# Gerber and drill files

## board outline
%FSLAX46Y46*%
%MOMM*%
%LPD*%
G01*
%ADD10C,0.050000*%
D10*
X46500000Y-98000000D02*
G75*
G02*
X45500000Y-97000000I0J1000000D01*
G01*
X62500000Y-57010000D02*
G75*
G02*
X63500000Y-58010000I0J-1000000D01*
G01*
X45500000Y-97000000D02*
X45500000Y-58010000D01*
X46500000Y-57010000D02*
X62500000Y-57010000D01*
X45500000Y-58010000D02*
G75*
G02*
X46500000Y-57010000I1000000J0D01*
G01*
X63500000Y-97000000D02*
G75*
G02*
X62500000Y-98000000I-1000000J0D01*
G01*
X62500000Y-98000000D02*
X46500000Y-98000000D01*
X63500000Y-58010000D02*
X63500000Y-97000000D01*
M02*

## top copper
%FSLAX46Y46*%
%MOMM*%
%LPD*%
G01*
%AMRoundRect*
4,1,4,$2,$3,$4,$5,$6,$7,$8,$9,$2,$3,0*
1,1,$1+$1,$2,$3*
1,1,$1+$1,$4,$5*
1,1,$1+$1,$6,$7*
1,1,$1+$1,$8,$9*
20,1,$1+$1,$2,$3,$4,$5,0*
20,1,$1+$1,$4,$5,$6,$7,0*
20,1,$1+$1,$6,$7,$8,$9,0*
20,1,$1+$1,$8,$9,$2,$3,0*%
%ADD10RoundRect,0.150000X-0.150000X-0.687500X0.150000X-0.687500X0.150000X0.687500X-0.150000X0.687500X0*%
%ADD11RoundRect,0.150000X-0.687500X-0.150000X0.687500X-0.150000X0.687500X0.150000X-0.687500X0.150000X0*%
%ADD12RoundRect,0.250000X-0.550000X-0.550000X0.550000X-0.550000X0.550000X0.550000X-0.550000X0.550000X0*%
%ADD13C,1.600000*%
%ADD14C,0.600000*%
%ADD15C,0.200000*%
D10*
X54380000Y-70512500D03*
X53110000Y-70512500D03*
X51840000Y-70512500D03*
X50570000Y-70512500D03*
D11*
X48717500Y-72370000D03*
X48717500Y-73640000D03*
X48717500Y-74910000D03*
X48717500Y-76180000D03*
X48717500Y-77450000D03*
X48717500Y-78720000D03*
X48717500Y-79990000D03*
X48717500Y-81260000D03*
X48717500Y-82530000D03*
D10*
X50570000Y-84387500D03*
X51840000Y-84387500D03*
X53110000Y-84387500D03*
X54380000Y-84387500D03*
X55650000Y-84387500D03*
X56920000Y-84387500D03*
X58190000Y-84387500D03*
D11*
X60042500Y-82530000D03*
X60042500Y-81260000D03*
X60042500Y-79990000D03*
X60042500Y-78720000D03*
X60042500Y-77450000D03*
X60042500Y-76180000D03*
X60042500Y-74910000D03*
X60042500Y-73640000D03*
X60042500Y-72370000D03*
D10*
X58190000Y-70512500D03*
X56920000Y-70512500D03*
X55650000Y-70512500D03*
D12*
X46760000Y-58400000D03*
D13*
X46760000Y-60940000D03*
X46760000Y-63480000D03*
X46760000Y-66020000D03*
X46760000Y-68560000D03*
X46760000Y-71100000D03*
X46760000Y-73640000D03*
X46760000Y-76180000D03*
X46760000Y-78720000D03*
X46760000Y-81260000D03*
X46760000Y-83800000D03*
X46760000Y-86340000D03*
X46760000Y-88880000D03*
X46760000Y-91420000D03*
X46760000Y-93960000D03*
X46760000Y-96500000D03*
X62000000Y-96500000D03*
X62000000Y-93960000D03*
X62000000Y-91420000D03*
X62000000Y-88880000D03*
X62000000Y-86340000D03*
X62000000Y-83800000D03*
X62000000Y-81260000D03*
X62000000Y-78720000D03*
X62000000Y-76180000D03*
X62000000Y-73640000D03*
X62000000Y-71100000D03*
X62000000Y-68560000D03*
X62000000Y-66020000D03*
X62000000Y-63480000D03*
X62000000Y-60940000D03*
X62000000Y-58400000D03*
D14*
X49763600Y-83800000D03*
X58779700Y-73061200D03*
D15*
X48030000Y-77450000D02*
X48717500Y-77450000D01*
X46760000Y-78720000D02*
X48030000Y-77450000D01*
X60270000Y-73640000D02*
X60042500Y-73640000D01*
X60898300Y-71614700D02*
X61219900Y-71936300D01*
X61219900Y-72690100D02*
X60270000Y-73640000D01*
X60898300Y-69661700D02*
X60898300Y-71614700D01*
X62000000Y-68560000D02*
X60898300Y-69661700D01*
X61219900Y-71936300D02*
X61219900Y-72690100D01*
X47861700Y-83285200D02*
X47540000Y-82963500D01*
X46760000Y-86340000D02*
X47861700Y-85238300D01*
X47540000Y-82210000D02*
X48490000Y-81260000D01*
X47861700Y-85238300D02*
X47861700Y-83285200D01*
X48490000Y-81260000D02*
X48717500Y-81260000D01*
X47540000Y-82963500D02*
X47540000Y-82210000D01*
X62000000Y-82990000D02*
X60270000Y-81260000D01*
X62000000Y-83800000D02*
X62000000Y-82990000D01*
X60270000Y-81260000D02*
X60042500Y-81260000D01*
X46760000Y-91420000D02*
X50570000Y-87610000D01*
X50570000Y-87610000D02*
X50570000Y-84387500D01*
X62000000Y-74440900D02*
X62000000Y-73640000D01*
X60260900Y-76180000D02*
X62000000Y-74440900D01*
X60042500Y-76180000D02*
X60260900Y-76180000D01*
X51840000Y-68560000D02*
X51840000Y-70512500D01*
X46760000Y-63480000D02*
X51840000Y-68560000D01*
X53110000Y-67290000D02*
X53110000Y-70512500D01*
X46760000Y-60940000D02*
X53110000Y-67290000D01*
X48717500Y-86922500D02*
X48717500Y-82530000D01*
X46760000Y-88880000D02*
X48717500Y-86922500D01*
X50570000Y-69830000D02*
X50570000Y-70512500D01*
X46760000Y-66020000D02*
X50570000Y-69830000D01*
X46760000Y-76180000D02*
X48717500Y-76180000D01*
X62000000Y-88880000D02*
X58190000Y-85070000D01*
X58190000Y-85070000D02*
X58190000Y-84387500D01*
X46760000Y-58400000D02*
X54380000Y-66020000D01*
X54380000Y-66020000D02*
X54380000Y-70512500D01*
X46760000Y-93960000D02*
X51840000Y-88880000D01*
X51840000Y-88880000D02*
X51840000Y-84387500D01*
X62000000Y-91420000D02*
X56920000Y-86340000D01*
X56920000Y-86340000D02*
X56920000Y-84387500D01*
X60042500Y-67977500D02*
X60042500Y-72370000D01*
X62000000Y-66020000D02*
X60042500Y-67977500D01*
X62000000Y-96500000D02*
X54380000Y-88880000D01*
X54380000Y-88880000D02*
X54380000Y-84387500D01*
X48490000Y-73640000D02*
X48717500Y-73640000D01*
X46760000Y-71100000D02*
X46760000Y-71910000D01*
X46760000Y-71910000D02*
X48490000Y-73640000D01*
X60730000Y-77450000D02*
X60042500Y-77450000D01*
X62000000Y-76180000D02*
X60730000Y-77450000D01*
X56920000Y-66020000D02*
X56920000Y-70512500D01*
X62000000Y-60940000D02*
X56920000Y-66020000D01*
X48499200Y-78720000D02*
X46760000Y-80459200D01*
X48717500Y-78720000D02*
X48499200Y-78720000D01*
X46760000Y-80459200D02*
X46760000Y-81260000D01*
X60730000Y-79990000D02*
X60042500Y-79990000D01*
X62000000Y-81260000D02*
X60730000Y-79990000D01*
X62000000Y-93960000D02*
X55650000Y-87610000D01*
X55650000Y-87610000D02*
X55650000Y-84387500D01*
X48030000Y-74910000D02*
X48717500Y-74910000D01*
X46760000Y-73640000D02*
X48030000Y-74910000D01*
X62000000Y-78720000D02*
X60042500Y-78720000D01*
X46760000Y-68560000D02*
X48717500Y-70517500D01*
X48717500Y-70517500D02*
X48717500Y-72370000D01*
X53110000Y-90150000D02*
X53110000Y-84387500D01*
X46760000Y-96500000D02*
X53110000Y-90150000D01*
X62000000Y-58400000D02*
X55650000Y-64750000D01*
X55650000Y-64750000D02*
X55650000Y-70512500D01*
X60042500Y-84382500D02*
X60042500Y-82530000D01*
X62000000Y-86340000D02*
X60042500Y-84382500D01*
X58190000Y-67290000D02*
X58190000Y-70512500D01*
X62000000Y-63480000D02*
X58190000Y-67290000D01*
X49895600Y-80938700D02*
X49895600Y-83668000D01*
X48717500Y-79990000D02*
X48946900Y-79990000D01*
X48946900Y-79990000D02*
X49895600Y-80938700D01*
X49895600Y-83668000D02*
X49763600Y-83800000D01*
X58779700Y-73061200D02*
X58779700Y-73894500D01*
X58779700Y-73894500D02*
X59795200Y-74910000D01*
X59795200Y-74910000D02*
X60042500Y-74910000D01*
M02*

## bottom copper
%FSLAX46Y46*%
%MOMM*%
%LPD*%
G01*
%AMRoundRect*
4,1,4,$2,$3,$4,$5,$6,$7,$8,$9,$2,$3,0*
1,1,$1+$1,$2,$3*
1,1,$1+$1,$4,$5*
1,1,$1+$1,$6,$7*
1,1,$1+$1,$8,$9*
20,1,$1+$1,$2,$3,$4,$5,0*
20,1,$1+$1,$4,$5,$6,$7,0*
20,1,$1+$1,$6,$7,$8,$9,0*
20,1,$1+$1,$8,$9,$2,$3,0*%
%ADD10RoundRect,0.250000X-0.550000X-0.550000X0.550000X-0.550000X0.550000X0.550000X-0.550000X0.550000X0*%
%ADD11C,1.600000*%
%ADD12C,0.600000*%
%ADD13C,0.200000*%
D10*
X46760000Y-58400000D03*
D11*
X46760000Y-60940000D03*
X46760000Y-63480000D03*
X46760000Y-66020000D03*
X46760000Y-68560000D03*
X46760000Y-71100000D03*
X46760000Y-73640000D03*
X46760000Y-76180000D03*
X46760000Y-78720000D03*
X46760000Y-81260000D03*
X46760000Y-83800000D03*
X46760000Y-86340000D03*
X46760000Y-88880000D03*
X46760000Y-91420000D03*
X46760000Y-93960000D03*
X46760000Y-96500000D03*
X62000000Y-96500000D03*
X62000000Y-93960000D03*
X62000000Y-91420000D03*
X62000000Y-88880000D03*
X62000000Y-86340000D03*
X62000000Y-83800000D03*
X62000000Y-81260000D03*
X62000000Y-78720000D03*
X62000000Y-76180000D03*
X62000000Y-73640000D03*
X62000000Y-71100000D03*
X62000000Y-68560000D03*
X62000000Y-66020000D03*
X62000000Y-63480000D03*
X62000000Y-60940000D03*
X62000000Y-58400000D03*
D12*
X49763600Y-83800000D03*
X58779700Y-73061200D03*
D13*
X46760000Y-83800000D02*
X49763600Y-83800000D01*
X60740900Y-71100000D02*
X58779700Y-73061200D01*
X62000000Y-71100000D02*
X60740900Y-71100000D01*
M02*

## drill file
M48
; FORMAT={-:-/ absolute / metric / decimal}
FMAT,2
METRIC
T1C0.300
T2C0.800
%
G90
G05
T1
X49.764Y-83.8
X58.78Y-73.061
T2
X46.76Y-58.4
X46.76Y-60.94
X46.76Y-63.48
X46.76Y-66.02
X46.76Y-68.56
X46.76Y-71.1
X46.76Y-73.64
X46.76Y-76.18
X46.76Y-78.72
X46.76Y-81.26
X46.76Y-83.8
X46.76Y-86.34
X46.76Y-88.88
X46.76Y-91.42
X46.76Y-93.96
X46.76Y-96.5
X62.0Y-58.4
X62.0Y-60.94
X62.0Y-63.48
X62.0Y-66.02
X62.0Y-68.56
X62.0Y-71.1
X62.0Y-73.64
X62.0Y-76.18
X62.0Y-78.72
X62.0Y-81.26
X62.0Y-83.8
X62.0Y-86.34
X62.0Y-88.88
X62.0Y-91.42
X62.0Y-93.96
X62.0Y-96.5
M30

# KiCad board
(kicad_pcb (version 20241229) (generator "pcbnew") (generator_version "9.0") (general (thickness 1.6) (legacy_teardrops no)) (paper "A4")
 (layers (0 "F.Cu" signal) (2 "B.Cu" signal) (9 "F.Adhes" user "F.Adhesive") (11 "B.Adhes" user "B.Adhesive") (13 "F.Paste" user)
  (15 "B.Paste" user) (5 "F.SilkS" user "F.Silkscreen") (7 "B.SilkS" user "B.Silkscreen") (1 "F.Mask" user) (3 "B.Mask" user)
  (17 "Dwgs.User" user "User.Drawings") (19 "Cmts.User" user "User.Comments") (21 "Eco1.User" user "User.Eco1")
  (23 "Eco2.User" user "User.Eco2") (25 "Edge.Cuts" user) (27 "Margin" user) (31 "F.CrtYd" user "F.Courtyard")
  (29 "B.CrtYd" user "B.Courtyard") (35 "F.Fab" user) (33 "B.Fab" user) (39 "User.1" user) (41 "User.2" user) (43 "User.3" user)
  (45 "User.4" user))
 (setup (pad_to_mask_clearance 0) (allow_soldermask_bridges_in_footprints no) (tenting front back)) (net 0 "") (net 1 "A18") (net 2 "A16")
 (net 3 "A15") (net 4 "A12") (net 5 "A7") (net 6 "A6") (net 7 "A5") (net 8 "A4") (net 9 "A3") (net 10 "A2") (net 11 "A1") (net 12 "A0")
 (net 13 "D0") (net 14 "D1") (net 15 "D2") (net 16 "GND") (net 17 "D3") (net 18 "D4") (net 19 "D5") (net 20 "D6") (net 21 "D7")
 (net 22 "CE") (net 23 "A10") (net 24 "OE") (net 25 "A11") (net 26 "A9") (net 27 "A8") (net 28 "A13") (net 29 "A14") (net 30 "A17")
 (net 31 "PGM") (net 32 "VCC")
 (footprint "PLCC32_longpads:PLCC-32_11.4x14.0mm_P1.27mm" (layer "F.Cu") (at 54.38 77.45)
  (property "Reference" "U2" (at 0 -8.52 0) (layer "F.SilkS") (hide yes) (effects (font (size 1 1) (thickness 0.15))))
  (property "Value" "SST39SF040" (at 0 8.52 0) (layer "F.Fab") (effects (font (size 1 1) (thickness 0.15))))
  (pad "1" smd roundrect (at 0 -6.9375) (size 0.6 1.675) (layers "F.Cu" "F.Mask" "F.Paste") (roundrect_rratio 0.25) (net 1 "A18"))
  (pad "2" smd roundrect (at -1.27 -6.9375) (size 0.6 1.675) (layers "F.Cu" "F.Mask" "F.Paste") (roundrect_rratio 0.25) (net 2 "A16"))
  (pad "3" smd roundrect (at -2.54 -6.9375) (size 0.6 1.675) (layers "F.Cu" "F.Mask" "F.Paste") (roundrect_rratio 0.25) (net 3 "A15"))
  (pad "4" smd roundrect (at -3.81 -6.9375) (size 0.6 1.675) (layers "F.Cu" "F.Mask" "F.Paste") (roundrect_rratio 0.25) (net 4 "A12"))
  (pad "5" smd roundrect (at -5.6625 -5.08) (size 1.675 0.6) (layers "F.Cu" "F.Mask" "F.Paste") (roundrect_rratio 0.25) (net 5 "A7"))
  (pad "6" smd roundrect (at -5.6625 -3.81) (size 1.675 0.6) (layers "F.Cu" "F.Mask" "F.Paste") (roundrect_rratio 0.25) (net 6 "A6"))
  (pad "7" smd roundrect (at -5.6625 -2.54) (size 1.675 0.6) (layers "F.Cu" "F.Mask" "F.Paste") (roundrect_rratio 0.25) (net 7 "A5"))
  (pad "8" smd roundrect (at -5.6625 -1.27) (size 1.675 0.6) (layers "F.Cu" "F.Mask" "F.Paste") (roundrect_rratio 0.25) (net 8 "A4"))
  (pad "9" smd roundrect (at -5.6625 0) (size 1.675 0.6) (layers "F.Cu" "F.Mask" "F.Paste") (roundrect_rratio 0.25) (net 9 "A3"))
  (pad "10" smd roundrect (at -5.6625 1.27) (size 1.675 0.6) (layers "F.Cu" "F.Mask" "F.Paste") (roundrect_rratio 0.25) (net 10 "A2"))
  (pad "11" smd roundrect (at -5.6625 2.54) (size 1.675 0.6) (layers "F.Cu" "F.Mask" "F.Paste") (roundrect_rratio 0.25) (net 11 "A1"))
  (pad "12" smd roundrect (at -5.6625 3.81) (size 1.675 0.6) (layers "F.Cu" "F.Mask" "F.Paste") (roundrect_rratio 0.25) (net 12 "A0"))
  (pad "13" smd roundrect (at -5.6625 5.08) (size 1.675 0.6) (layers "F.Cu" "F.Mask" "F.Paste") (roundrect_rratio 0.25) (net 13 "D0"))
  (pad "14" smd roundrect (at -3.81 6.9375) (size 0.6 1.675) (layers "F.Cu" "F.Mask" "F.Paste") (roundrect_rratio 0.25) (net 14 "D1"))
  (pad "15" smd roundrect (at -2.54 6.9375) (size 0.6 1.675) (layers "F.Cu" "F.Mask" "F.Paste") (roundrect_rratio 0.25) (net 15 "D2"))
  (pad "16" smd roundrect (at -1.27 6.9375) (size 0.6 1.675) (layers "F.Cu" "F.Mask" "F.Paste") (roundrect_rratio 0.25) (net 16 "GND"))
  (pad "17" smd roundrect (at 0 6.9375) (size 0.6 1.675) (layers "F.Cu" "F.Mask" "F.Paste") (roundrect_rratio 0.25) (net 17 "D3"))
  (pad "18" smd roundrect (at 1.27 6.9375) (size 0.6 1.675) (layers "F.Cu" "F.Mask" "F.Paste") (roundrect_rratio 0.25) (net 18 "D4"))
  (pad "19" smd roundrect (at 2.54 6.9375) (size 0.6 1.675) (layers "F.Cu" "F.Mask" "F.Paste") (roundrect_rratio 0.25) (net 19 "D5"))
  (pad "20" smd roundrect (at 3.81 6.9375) (size 0.6 1.675) (layers "F.Cu" "F.Mask" "F.Paste") (roundrect_rratio 0.25) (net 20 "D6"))
  (pad "21" smd roundrect (at 5.6625 5.08) (size 1.675 0.6) (layers "F.Cu" "F.Mask" "F.Paste") (roundrect_rratio 0.25) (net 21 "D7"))
  (pad "22" smd roundrect (at 5.6625 3.81) (size 1.675 0.6) (layers "F.Cu" "F.Mask" "F.Paste") (roundrect_rratio 0.25) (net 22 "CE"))
  (pad "23" smd roundrect (at 5.6625 2.54) (size 1.675 0.6) (layers "F.Cu" "F.Mask" "F.Paste") (roundrect_rratio 0.25) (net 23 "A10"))
  (pad "24" smd roundrect (at 5.6625 1.27) (size 1.675 0.6) (layers "F.Cu" "F.Mask" "F.Paste") (roundrect_rratio 0.25) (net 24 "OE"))
  (pad "25" smd roundrect (at 5.6625 0) (size 1.675 0.6) (layers "F.Cu" "F.Mask" "F.Paste") (roundrect_rratio 0.25) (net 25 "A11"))
  (pad "26" smd roundrect (at 5.6625 -1.27) (size 1.675 0.6) (layers "F.Cu" "F.Mask" "F.Paste") (roundrect_rratio 0.25) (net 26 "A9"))
  (pad "27" smd roundrect (at 5.6625 -2.54) (size 1.675 0.6) (layers "F.Cu" "F.Mask" "F.Paste") (roundrect_rratio 0.25) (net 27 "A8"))
  (pad "28" smd roundrect (at 5.6625 -3.81) (size 1.675 0.6) (layers "F.Cu" "F.Mask" "F.Paste") (roundrect_rratio 0.25) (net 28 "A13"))
  (pad "29" smd roundrect (at 5.6625 -5.08) (size 1.675 0.6) (layers "F.Cu" "F.Mask" "F.Paste") (roundrect_rratio 0.25) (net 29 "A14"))
  (pad "30" smd roundrect (at 3.81 -6.9375) (size 0.6 1.675) (layers "F.Cu" "F.Mask" "F.Paste") (roundrect_rratio 0.25) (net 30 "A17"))
  (pad "31" smd roundrect (at 2.54 -6.9375) (size 0.6 1.675) (layers "F.Cu" "F.Mask" "F.Paste") (roundrect_rratio 0.25) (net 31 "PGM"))
  (pad "32" smd roundrect (at 1.27 -6.9375) (size 0.6 1.675) (layers "F.Cu" "F.Mask" "F.Paste") (roundrect_rratio 0.25) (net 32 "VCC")))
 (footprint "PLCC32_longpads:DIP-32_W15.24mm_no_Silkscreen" (layer "F.Cu") (at 46.76 58.4)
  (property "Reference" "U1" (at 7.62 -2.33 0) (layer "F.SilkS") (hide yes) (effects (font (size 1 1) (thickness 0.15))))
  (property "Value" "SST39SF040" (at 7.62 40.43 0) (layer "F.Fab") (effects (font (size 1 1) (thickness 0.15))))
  (pad "1" thru_hole roundrect (at 0 0) (size 1.6 1.6) (drill 0.8) (layers "*.Cu" "*.Mask") (remove_unused_layers no)
   (roundrect_rratio 0.15625) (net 1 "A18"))
  (pad "2" thru_hole circle (at 0 2.54) (size 1.6 1.6) (drill 0.8) (layers "*.Cu" "*.Mask") (remove_unused_layers no) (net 2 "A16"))
  (pad "3" thru_hole circle (at 0 5.08) (size 1.6 1.6) (drill 0.8) (layers "*.Cu" "*.Mask") (remove_unused_layers no) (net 3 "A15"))
  (pad "4" thru_hole circle (at 0 7.62) (size 1.6 1.6) (drill 0.8) (layers "*.Cu" "*.Mask") (remove_unused_layers no) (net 4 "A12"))
  (pad "5" thru_hole circle (at 0 10.16) (size 1.6 1.6) (drill 0.8) (layers "*.Cu" "*.Mask") (remove_unused_layers no) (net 5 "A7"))
  (pad "6" thru_hole circle (at 0 12.7) (size 1.6 1.6) (drill 0.8) (layers "*.Cu" "*.Mask") (remove_unused_layers no) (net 6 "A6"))
  (pad "7" thru_hole circle (at 0 15.24) (size 1.6 1.6) (drill 0.8) (layers "*.Cu" "*.Mask") (remove_unused_layers no) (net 7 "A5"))
  (pad "8" thru_hole circle (at 0 17.78) (size 1.6 1.6) (drill 0.8) (layers "*.Cu" "*.Mask") (remove_unused_layers no) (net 8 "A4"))
  (pad "9" thru_hole circle (at 0 20.32) (size 1.6 1.6) (drill 0.8) (layers "*.Cu" "*.Mask") (remove_unused_layers no) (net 9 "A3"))
  (pad "10" thru_hole circle (at 0 22.86) (size 1.6 1.6) (drill 0.8) (layers "*.Cu" "*.Mask") (remove_unused_layers no) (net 10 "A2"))
  (pad "11" thru_hole circle (at 0 25.4) (size 1.6 1.6) (drill 0.8) (layers "*.Cu" "*.Mask") (remove_unused_layers no) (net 11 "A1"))
  (pad "12" thru_hole circle (at 0 27.94) (size 1.6 1.6) (drill 0.8) (layers "*.Cu" "*.Mask") (remove_unused_layers no) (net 12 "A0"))
  (pad "13" thru_hole circle (at 0 30.48) (size 1.6 1.6) (drill 0.8) (layers "*.Cu" "*.Mask") (remove_unused_layers no) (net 13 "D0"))
  (pad "14" thru_hole circle (at 0 33.02) (size 1.6 1.6) (drill 0.8) (layers "*.Cu" "*.Mask") (remove_unused_layers no) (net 14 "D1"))
  (pad "15" thru_hole circle (at 0 35.56) (size 1.6 1.6) (drill 0.8) (layers "*.Cu" "*.Mask") (remove_unused_layers no) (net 15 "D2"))
  (pad "16" thru_hole circle (at 0 38.1) (size 1.6 1.6) (drill 0.8) (layers "*.Cu" "*.Mask") (remove_unused_layers no) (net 16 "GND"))
  (pad "17" thru_hole circle (at 15.24 38.1) (size 1.6 1.6) (drill 0.8) (layers "*.Cu" "*.Mask") (remove_unused_layers no) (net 17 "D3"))
  (pad "18" thru_hole circle (at 15.24 35.56) (size 1.6 1.6) (drill 0.8) (layers "*.Cu" "*.Mask") (remove_unused_layers no) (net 18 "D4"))
  (pad "19" thru_hole circle (at 15.24 33.02) (size 1.6 1.6) (drill 0.8) (layers "*.Cu" "*.Mask") (remove_unused_layers no) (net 19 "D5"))
  (pad "20" thru_hole circle (at 15.24 30.48) (size 1.6 1.6) (drill 0.8) (layers "*.Cu" "*.Mask") (remove_unused_layers no) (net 20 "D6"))
  (pad "21" thru_hole circle (at 15.24 27.94) (size 1.6 1.6) (drill 0.8) (layers "*.Cu" "*.Mask") (remove_unused_layers no) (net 21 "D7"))
  (pad "22" thru_hole circle (at 15.24 25.4) (size 1.6 1.6) (drill 0.8) (layers "*.Cu" "*.Mask") (remove_unused_layers no) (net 22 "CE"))
  (pad "23" thru_hole circle (at 15.24 22.86) (size 1.6 1.6) (drill 0.8) (layers "*.Cu" "*.Mask") (remove_unused_layers no) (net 23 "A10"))
  (pad "24" thru_hole circle (at 15.24 20.32) (size 1.6 1.6) (drill 0.8) (layers "*.Cu" "*.Mask") (remove_unused_layers no) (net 24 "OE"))
  (pad "25" thru_hole circle (at 15.24 17.78) (size 1.6 1.6) (drill 0.8) (layers "*.Cu" "*.Mask") (remove_unused_layers no) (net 25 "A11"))
  (pad "26" thru_hole circle (at 15.24 15.24) (size 1.6 1.6) (drill 0.8) (layers "*.Cu" "*.Mask") (remove_unused_layers no) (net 26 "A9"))
  (pad "27" thru_hole circle (at 15.24 12.7) (size 1.6 1.6) (drill 0.8) (layers "*.Cu" "*.Mask") (remove_unused_layers no) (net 27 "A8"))
  (pad "28" thru_hole circle (at 15.24 10.16) (size 1.6 1.6) (drill 0.8) (layers "*.Cu" "*.Mask") (remove_unused_layers no) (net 28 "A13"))
  (pad "29" thru_hole circle (at 15.24 7.62) (size 1.6 1.6) (drill 0.8) (layers "*.Cu" "*.Mask") (remove_unused_layers no) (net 29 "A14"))
  (pad "30" thru_hole circle (at 15.24 5.08) (size 1.6 1.6) (drill 0.8) (layers "*.Cu" "*.Mask") (remove_unused_layers no) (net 30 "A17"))
  (pad "31" thru_hole circle (at 15.24 2.54) (size 1.6 1.6) (drill 0.8) (layers "*.Cu" "*.Mask") (remove_unused_layers no) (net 31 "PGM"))
  (pad "32" thru_hole circle (at 15.24 0) (size 1.6 1.6) (drill 0.8) (layers "*.Cu" "*.Mask") (remove_unused_layers no) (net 32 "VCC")))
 (gr_arc (start 46.5 98) (mid 45.792893 97.707107) (end 45.5 97) (stroke (width 0.05) (type default)) (layer "Edge.Cuts"))
 (gr_arc (start 62.5 57.01) (mid 63.207107 57.302893) (end 63.5 58.01) (stroke (width 0.05) (type default)) (layer "Edge.Cuts"))
 (gr_line (start 45.5 97) (end 45.5 58.01) (stroke (width 0.05) (type default)) (layer "Edge.Cuts"))
 (gr_line (start 46.5 57.01) (end 62.5 57.01) (stroke (width 0.05) (type default)) (layer "Edge.Cuts"))
 (gr_arc (start 45.5 58.01) (mid 45.792893 57.302893) (end 46.5 57.01) (stroke (width 0.05) (type default)) (layer "Edge.Cuts"))
 (gr_arc (start 63.5 97) (mid 63.207107 97.707107) (end 62.5 98) (stroke (width 0.05) (type default)) (layer "Edge.Cuts"))
 (gr_line (start 62.5 98) (end 46.5 98) (stroke (width 0.05) (type default)) (layer "Edge.Cuts"))
 (gr_line (start 63.5 58.01) (end 63.5 97) (stroke (width 0.05) (type default)) (layer "Edge.Cuts"))
 (segment (start 48.03 77.45) (end 48.7175 77.45) (width 0.2) (layer "F.Cu") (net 9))
 (segment (start 46.76 78.72) (end 48.03 77.45) (width 0.2) (layer "F.Cu") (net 9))
 (segment (start 60.27 73.64) (end 60.0425 73.64) (width 0.2) (layer "F.Cu") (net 28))
 (segment (start 60.8983 71.6147) (end 61.2199 71.9363) (width 0.2) (layer "F.Cu") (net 28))
 (segment (start 61.2199 72.6901) (end 60.27 73.64) (width 0.2) (layer "F.Cu") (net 28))
 (segment (start 60.8983 69.6617) (end 60.8983 71.6147) (width 0.2) (layer "F.Cu") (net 28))
 (segment (start 62 68.56) (end 60.8983 69.6617) (width 0.2) (layer "F.Cu") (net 28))
 (segment (start 61.2199 71.9363) (end 61.2199 72.6901) (width 0.2) (layer "F.Cu") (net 28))
 (segment (start 47.8617 83.2852) (end 47.54 82.9635) (width 0.2) (layer "F.Cu") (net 12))
 (segment (start 46.76 86.34) (end 47.8617 85.2383) (width 0.2) (layer "F.Cu") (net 12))
 (segment (start 47.54 82.21) (end 48.49 81.26) (width 0.2) (layer "F.Cu") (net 12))
 (segment (start 47.8617 85.2383) (end 47.8617 83.2852) (width 0.2) (layer "F.Cu") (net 12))
 (segment (start 48.49 81.26) (end 48.7175 81.26) (width 0.2) (layer "F.Cu") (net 12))
 (segment (start 47.54 82.9635) (end 47.54 82.21) (width 0.2) (layer "F.Cu") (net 12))
 (segment (start 62 82.99) (end 60.27 81.26) (width 0.2) (layer "F.Cu") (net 22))
 (segment (start 62 83.8) (end 62 82.99) (width 0.2) (layer "F.Cu") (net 22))
 (segment (start 60.27 81.26) (end 60.0425 81.26) (width 0.2) (layer "F.Cu") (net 22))
 (segment (start 46.76 91.42) (end 50.57 87.61) (width 0.2) (layer "F.Cu") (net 14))
 (segment (start 50.57 87.61) (end 50.57 84.3875) (width 0.2) (layer "F.Cu") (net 14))
 (segment (start 62 74.4409) (end 62 73.64) (width 0.2) (layer "F.Cu") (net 26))
 (segment (start 60.2609 76.18) (end 62 74.4409) (width 0.2) (layer "F.Cu") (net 26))
 (segment (start 60.0425 76.18) (end 60.2609 76.18) (width 0.2) (layer "F.Cu") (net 26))
 (segment (start 51.84 68.56) (end 51.84 70.5125) (width 0.2) (layer "F.Cu") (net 3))
 (segment (start 46.76 63.48) (end 51.84 68.56) (width 0.2) (layer "F.Cu") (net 3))
 (segment (start 53.11 67.29) (end 53.11 70.5125) (width 0.2) (layer "F.Cu") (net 2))
 (segment (start 46.76 60.94) (end 53.11 67.29) (width 0.2) (layer "F.Cu") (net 2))
 (segment (start 48.7175 86.9225) (end 48.7175 82.53) (width 0.2) (layer "F.Cu") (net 13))
 (segment (start 46.76 88.88) (end 48.7175 86.9225) (width 0.2) (layer "F.Cu") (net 13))
 (segment (start 50.57 69.83) (end 50.57 70.5125) (width 0.2) (layer "F.Cu") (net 4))
 (segment (start 46.76 66.02) (end 50.57 69.83) (width 0.2) (layer "F.Cu") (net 4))
 (segment (start 46.76 76.18) (end 48.7175 76.18) (width 0.2) (layer "F.Cu") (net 8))
 (segment (start 62 88.88) (end 58.19 85.07) (width 0.2) (layer "F.Cu") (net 20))
 (segment (start 58.19 85.07) (end 58.19 84.3875) (width 0.2) (layer "F.Cu") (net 20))
 (segment (start 46.76 58.4) (end 54.38 66.02) (width 0.2) (layer "F.Cu") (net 1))
 (segment (start 54.38 66.02) (end 54.38 70.5125) (width 0.2) (layer "F.Cu") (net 1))
 (segment (start 46.76 93.96) (end 51.84 88.88) (width 0.2) (layer "F.Cu") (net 15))
 (segment (start 51.84 88.88) (end 51.84 84.3875) (width 0.2) (layer "F.Cu") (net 15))
 (segment (start 62 91.42) (end 56.92 86.34) (width 0.2) (layer "F.Cu") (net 19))
 (segment (start 56.92 86.34) (end 56.92 84.3875) (width 0.2) (layer "F.Cu") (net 19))
 (segment (start 60.0425 67.9775) (end 60.0425 72.37) (width 0.2) (layer "F.Cu") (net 29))
 (segment (start 62 66.02) (end 60.0425 67.9775) (width 0.2) (layer "F.Cu") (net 29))
 (segment (start 62 96.5) (end 54.38 88.88) (width 0.2) (layer "F.Cu") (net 17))
 (segment (start 54.38 88.88) (end 54.38 84.3875) (width 0.2) (layer "F.Cu") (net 17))
 (segment (start 48.49 73.64) (end 48.7175 73.64) (width 0.2) (layer "F.Cu") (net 6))
 (segment (start 46.76 71.1) (end 46.76 71.91) (width 0.2) (layer "F.Cu") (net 6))
 (segment (start 46.76 71.91) (end 48.49 73.64) (width 0.2) (layer "F.Cu") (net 6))
 (segment (start 60.73 77.45) (end 60.0425 77.45) (width 0.2) (layer "F.Cu") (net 25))
 (segment (start 62 76.18) (end 60.73 77.45) (width 0.2) (layer "F.Cu") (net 25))
 (segment (start 56.92 66.02) (end 56.92 70.5125) (width 0.2) (layer "F.Cu") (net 31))
 (segment (start 62 60.94) (end 56.92 66.02) (width 0.2) (layer "F.Cu") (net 31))
 (segment (start 48.4992 78.72) (end 46.76 80.4592) (width 0.2) (layer "F.Cu") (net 10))
 (segment (start 48.7175 78.72) (end 48.4992 78.72) (width 0.2) (layer "F.Cu") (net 10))
 (segment (start 46.76 80.4592) (end 46.76 81.26) (width 0.2) (layer "F.Cu") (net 10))
 (segment (start 60.73 79.99) (end 60.0425 79.99) (width 0.2) (layer "F.Cu") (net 23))
 (segment (start 62 81.26) (end 60.73 79.99) (width 0.2) (layer "F.Cu") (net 23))
 (segment (start 62 93.96) (end 55.65 87.61) (width 0.2) (layer "F.Cu") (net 18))
 (segment (start 55.65 87.61) (end 55.65 84.3875) (width 0.2) (layer "F.Cu") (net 18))
 (segment (start 48.03 74.91) (end 48.7175 74.91) (width 0.2) (layer "F.Cu") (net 7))
 (segment (start 46.76 73.64) (end 48.03 74.91) (width 0.2) (layer "F.Cu") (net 7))
 (segment (start 62 78.72) (end 60.0425 78.72) (width 0.2) (layer "F.Cu") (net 24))
 (segment (start 46.76 68.56) (end 48.7175 70.5175) (width 0.2) (layer "F.Cu") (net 5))
 (segment (start 48.7175 70.5175) (end 48.7175 72.37) (width 0.2) (layer "F.Cu") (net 5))
 (segment (start 53.11 90.15) (end 53.11 84.3875) (width 0.2) (layer "F.Cu") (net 16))
 (segment (start 46.76 96.5) (end 53.11 90.15) (width 0.2) (layer "F.Cu") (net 16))
 (segment (start 62 58.4) (end 55.65 64.75) (width 0.2) (layer "F.Cu") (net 32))
 (segment (start 55.65 64.75) (end 55.65 70.5125) (width 0.2) (layer "F.Cu") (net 32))
 (segment (start 60.0425 84.3825) (end 60.0425 82.53) (width 0.2) (layer "F.Cu") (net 21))
 (segment (start 62 86.34) (end 60.0425 84.3825) (width 0.2) (layer "F.Cu") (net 21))
 (segment (start 58.19 67.29) (end 58.19 70.5125) (width 0.2) (layer "F.Cu") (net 30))
 (segment (start 62 63.48) (end 58.19 67.29) (width 0.2) (layer "F.Cu") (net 30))
 (segment (start 49.8956 80.9387) (end 49.8956 83.668) (width 0.2) (layer "F.Cu") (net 11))
 (segment (start 48.7175 79.99) (end 48.9469 79.99) (width 0.2) (layer "F.Cu") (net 11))
 (segment (start 48.9469 79.99) (end 49.8956 80.9387) (width 0.2) (layer "F.Cu") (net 11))
 (segment (start 49.8956 83.668) (end 49.7636 83.8) (width 0.2) (layer "F.Cu") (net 11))
 (via (at 49.7636 83.8) (size 0.6) (drill 0.3) (layers "F.Cu" "B.Cu") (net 11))
 (segment (start 46.76 83.8) (end 49.7636 83.8) (width 0.2) (layer "B.Cu") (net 11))
 (segment (start 58.7797 73.0612) (end 58.7797 73.8945) (width 0.2) (layer "F.Cu") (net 27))
 (segment (start 58.7797 73.8945) (end 59.7952 74.91) (width 0.2) (layer "F.Cu") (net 27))
 (segment (start 59.7952 74.91) (end 60.0425 74.91) (width 0.2) (layer "F.Cu") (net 27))
 (via (at 58.7797 73.0612) (size 0.6) (drill 0.3) (layers "F.Cu" "B.Cu") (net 27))
 (segment (start 60.7409 71.1) (end 58.7797 73.0612) (width 0.2) (layer "B.Cu") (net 27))
 (segment (start 62 71.1) (end 60.7409 71.1) (width 0.2) (layer "B.Cu") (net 27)))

